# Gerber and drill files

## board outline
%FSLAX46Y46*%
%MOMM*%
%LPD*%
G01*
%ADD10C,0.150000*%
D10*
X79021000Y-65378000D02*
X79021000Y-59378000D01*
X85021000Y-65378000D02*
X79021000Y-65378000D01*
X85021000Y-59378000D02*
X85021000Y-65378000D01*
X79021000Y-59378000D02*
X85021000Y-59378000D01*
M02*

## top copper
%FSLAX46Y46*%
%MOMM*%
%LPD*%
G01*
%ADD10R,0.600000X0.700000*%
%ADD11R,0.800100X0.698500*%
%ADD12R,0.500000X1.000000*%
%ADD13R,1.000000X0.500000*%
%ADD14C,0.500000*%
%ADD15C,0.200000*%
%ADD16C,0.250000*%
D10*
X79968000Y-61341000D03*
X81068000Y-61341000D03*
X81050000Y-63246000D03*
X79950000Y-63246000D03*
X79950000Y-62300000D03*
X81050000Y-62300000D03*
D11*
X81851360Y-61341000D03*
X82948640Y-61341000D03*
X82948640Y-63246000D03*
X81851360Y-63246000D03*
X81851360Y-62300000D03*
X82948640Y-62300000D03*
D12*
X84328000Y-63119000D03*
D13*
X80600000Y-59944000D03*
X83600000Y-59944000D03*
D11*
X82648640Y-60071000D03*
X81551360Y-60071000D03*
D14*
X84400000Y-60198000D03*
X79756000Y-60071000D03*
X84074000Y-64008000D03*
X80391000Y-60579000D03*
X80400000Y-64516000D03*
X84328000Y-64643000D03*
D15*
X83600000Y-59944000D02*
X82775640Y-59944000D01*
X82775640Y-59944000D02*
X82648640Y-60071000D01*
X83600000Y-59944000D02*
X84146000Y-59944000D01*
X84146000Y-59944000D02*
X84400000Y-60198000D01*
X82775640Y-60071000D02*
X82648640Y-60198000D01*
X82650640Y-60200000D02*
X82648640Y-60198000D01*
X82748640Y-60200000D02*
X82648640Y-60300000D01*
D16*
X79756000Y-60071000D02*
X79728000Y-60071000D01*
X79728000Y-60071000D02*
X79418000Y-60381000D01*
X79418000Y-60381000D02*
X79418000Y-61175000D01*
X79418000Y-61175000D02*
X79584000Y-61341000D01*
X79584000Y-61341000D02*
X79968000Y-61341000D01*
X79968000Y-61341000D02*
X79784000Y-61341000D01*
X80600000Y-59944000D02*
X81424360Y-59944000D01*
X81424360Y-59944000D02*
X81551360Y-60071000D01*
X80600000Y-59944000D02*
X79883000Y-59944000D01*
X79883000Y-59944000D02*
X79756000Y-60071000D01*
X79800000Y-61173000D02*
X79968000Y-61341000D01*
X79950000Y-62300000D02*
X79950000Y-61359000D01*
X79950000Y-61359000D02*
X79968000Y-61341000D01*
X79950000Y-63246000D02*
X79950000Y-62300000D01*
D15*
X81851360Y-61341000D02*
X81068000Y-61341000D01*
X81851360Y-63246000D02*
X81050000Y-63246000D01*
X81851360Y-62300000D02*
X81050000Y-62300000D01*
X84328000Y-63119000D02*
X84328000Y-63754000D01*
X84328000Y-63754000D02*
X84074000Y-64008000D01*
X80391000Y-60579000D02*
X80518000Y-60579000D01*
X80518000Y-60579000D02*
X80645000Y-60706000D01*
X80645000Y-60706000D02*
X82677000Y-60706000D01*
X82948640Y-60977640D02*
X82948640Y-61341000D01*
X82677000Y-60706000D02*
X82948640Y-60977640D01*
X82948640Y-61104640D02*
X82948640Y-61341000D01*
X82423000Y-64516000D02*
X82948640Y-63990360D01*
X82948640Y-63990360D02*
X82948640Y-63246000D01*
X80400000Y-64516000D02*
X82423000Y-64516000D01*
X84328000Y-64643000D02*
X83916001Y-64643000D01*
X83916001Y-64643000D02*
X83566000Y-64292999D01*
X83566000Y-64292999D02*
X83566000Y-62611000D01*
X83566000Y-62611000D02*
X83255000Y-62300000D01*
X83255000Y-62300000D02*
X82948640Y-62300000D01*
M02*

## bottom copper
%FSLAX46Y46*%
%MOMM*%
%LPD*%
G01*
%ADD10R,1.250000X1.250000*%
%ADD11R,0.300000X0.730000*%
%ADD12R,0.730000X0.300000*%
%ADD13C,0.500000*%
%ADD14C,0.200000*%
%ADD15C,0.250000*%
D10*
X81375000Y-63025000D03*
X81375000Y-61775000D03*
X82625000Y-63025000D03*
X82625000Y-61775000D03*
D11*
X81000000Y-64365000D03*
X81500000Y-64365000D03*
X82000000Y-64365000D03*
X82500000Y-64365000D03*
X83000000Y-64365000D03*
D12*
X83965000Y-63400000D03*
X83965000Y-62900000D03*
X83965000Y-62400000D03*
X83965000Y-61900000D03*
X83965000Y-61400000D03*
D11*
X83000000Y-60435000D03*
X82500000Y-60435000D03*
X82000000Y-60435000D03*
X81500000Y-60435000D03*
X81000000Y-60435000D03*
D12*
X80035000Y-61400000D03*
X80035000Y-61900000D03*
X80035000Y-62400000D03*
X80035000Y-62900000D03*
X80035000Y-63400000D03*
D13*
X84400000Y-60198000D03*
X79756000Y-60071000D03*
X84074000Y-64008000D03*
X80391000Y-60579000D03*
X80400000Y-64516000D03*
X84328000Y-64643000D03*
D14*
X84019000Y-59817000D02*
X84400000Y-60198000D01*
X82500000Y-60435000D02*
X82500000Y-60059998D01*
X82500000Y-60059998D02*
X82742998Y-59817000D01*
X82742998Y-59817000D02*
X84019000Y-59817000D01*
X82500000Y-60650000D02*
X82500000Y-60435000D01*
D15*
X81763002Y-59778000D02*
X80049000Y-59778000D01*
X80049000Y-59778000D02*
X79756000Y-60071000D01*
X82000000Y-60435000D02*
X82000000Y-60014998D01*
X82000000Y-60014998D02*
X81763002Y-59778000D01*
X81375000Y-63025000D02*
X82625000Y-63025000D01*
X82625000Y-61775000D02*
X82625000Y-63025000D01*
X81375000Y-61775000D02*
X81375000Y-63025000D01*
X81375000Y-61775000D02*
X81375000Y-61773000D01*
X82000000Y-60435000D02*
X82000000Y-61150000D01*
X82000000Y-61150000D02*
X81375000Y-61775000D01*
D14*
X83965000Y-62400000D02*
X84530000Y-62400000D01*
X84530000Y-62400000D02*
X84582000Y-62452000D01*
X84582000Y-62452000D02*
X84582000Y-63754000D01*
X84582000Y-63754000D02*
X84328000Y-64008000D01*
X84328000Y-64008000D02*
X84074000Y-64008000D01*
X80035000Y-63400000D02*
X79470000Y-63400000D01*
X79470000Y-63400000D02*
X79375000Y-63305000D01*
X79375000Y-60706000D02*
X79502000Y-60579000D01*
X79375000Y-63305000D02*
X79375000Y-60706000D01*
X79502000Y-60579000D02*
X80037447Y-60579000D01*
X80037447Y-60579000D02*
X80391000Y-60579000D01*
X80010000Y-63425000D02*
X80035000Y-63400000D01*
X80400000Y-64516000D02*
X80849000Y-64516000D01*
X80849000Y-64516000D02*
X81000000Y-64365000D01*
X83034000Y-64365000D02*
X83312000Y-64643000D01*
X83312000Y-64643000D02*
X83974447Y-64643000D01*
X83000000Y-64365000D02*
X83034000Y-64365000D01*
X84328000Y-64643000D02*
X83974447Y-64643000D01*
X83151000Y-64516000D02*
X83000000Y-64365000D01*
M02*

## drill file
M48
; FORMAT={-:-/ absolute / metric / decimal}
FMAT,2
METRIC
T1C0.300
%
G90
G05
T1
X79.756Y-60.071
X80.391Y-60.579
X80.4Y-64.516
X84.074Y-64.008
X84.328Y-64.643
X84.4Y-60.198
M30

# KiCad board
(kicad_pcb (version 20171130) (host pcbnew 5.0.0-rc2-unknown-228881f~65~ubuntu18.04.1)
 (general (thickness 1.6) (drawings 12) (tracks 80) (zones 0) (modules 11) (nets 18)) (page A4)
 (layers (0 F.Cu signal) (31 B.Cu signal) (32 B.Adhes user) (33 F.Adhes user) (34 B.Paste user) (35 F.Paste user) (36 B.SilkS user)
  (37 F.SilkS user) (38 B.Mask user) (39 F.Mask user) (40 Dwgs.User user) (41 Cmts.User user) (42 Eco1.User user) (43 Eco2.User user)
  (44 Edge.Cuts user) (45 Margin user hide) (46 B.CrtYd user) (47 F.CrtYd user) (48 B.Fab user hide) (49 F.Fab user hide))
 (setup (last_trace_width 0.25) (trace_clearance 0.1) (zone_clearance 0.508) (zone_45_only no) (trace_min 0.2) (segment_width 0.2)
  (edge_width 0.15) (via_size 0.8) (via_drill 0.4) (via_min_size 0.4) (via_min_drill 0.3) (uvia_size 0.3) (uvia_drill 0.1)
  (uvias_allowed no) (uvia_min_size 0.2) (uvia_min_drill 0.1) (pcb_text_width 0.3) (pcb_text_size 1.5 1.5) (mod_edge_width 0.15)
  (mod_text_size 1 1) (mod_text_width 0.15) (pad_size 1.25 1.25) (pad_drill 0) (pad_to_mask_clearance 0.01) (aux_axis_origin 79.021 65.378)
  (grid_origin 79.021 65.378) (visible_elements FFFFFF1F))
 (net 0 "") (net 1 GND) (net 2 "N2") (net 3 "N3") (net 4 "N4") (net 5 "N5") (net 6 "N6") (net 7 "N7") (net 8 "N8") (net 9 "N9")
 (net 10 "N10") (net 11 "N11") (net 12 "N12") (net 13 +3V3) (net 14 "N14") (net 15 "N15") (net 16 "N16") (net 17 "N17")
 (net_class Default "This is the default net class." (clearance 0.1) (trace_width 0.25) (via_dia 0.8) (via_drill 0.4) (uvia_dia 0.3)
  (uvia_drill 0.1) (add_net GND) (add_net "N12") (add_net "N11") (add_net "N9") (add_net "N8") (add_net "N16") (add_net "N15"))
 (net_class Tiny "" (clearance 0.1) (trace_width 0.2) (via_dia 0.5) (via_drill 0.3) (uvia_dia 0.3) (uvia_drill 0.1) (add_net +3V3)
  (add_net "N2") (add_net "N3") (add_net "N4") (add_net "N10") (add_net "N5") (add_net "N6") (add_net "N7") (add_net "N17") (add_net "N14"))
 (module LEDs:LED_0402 (layer F.Cu) (at 80.518 61.341)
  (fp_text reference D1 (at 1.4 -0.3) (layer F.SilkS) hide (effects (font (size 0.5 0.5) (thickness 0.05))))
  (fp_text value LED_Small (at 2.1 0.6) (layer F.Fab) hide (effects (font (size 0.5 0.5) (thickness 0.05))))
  (pad 1 smd rect (at -0.55 0 180) (size 0.6 0.7) (layers F.Cu F.Paste F.Mask) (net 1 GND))
  (pad 2 smd rect (at 0.55 0 180) (size 0.6 0.7) (layers F.Cu F.Paste F.Mask) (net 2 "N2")))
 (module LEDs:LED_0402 (layer F.Cu) (at 80.5 63.246)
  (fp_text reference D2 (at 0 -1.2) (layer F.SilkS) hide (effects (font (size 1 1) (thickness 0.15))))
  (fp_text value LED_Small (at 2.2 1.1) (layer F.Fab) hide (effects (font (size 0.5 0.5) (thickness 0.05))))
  (pad 2 smd rect (at 0.55 0 180) (size 0.6 0.7) (layers F.Cu F.Paste F.Mask) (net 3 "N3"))
  (pad 1 smd rect (at -0.55 0 180) (size 0.6 0.7) (layers F.Cu F.Paste F.Mask) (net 1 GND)))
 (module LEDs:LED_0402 (layer F.Cu) (at 80.5 62.3)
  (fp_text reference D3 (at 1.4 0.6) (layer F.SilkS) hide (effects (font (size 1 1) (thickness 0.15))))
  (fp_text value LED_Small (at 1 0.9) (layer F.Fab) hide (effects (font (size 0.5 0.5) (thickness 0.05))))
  (pad 1 smd rect (at -0.55 0 180) (size 0.6 0.7) (layers F.Cu F.Paste F.Mask) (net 1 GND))
  (pad 2 smd rect (at 0.55 0 180) (size 0.6 0.7) (layers F.Cu F.Paste F.Mask) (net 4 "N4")))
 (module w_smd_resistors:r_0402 (layer F.Cu) (at 82.4 61.341 180)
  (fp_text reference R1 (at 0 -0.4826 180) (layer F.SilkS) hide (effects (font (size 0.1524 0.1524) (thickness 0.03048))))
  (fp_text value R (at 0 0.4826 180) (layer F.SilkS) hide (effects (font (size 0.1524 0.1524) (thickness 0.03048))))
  (pad 1 smd rect (at 0.54864 0 180) (size 0.8001 0.6985) (layers F.Cu F.Paste F.Mask) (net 2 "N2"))
  (pad 2 smd rect (at -0.54864 0 180) (size 0.8001 0.6985) (layers F.Cu F.Paste F.Mask) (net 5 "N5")))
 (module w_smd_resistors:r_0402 (layer F.Cu) (at 82.4 63.246 180)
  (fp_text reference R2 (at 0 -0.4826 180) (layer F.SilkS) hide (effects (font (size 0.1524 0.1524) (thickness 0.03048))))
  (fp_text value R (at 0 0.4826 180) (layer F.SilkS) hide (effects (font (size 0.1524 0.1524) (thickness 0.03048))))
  (pad 2 smd rect (at -0.54864 0 180) (size 0.8001 0.6985) (layers F.Cu F.Paste F.Mask) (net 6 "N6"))
  (pad 1 smd rect (at 0.54864 0 180) (size 0.8001 0.6985) (layers F.Cu F.Paste F.Mask) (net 3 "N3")))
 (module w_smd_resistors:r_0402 (layer F.Cu) (at 82.4 62.3 180)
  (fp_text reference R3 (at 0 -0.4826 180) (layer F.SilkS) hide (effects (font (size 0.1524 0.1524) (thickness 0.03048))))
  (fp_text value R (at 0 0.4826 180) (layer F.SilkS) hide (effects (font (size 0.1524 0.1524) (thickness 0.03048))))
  (pad 1 smd rect (at 0.54864 0 180) (size 0.8001 0.6985) (layers F.Cu F.Paste F.Mask) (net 4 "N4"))
  (pad 2 smd rect (at -0.54864 0 180) (size 0.8001 0.6985) (layers F.Cu F.Paste F.Mask) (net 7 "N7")))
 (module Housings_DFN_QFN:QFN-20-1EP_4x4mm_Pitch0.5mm (layer B.Cu) (at 82 62.4)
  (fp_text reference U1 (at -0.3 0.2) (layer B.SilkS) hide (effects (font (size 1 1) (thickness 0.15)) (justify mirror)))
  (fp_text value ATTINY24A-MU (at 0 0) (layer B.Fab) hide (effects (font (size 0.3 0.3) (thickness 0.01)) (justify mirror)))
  (pad 21 smd rect (at -0.625 0.625) (size 1.25 1.25) (layers B.Cu B.Paste B.Mask) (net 1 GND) (solder_paste_margin_ratio -0.2))
  (pad 21 smd rect (at -0.625 -0.625) (size 1.25 1.25) (layers B.Cu B.Paste B.Mask) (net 1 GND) (solder_paste_margin_ratio -0.2))
  (pad 21 smd rect (at 0.625 0.625) (size 1.25 1.25) (layers B.Cu B.Paste B.Mask) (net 1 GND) (solder_paste_margin_ratio -0.2))
  (pad 21 smd rect (at 0.625 -0.625) (size 1.25 1.25) (layers B.Cu B.Paste B.Mask) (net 1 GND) (solder_paste_margin_ratio -0.2))
  (pad 20 smd rect (at -1 1.965 270) (size 0.73 0.3) (layers B.Cu B.Paste B.Mask) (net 6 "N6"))
  (pad 19 smd rect (at -0.5 1.965 270) (size 0.73 0.3) (layers B.Cu B.Paste B.Mask))
  (pad 18 smd rect (at 0 1.965 270) (size 0.73 0.3) (layers B.Cu B.Paste B.Mask))
  (pad 17 smd rect (at 0.5 1.965 270) (size 0.73 0.3) (layers B.Cu B.Paste B.Mask))
  (pad 16 smd rect (at 1 1.965 270) (size 0.73 0.3) (layers B.Cu B.Paste B.Mask) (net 7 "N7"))
  (pad 15 smd rect (at 1.965 1) (size 0.73 0.3) (layers B.Cu B.Paste B.Mask) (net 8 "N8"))
  (pad 14 smd rect (at 1.965 0.5) (size 0.73 0.3) (layers B.Cu B.Paste B.Mask) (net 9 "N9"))
  (pad 13 smd rect (at 1.965 0) (size 0.73 0.3) (layers B.Cu B.Paste B.Mask) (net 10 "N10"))
  (pad 12 smd rect (at 1.965 -0.5) (size 0.73 0.3) (layers B.Cu B.Paste B.Mask) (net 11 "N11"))
  (pad 11 smd rect (at 1.965 -1) (size 0.73 0.3) (layers B.Cu B.Paste B.Mask) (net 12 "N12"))
  (pad 10 smd rect (at 1 -1.965 270) (size 0.73 0.3) (layers B.Cu B.Paste B.Mask))
  (pad 9 smd rect (at 0.5 -1.965 270) (size 0.73 0.3) (layers B.Cu B.Paste B.Mask) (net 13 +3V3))
  (pad 8 smd rect (at 0 -1.965 270) (size 0.73 0.3) (layers B.Cu B.Paste B.Mask) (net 1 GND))
  (pad 7 smd rect (at -0.5 -1.965 270) (size 0.73 0.3) (layers B.Cu B.Paste B.Mask))
  (pad 6 smd rect (at -1 -1.965 270) (size 0.73 0.3) (layers B.Cu B.Paste B.Mask))
  (pad 5 smd rect (at -1.965 -1) (size 0.73 0.3) (layers B.Cu B.Paste B.Mask) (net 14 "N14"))
  (pad 4 smd rect (at -1.965 -0.5) (size 0.73 0.3) (layers B.Cu B.Paste B.Mask) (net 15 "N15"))
  (pad 3 smd rect (at -1.965 0) (size 0.73 0.3) (layers B.Cu B.Paste B.Mask) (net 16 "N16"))
  (pad 2 smd rect (at -1.965 0.5) (size 0.73 0.3) (layers B.Cu B.Paste B.Mask) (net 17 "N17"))
  (pad 1 smd rect (at -1.965 1) (size 0.73 0.3) (layers B.Cu B.Paste B.Mask) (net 5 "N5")))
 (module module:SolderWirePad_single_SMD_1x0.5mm (layer F.Cu) (at 84.328 63.119 90)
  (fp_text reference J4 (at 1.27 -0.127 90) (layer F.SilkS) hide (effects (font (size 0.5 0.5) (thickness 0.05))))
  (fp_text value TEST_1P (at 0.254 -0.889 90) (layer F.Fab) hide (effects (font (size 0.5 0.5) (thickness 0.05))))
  (pad 1 smd rect (at 0 0 90) (size 1 0.5) (layers F.Cu F.Paste F.Mask) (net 10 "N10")))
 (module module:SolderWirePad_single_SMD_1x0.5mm (layer F.Cu) (at 80.6 59.944 180)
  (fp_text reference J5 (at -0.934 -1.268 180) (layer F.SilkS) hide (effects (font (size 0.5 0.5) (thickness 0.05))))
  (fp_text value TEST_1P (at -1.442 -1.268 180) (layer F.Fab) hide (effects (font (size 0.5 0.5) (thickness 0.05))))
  (pad 1 smd rect (at 0 0 180) (size 1 0.5) (layers F.Cu F.Paste F.Mask) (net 1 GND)))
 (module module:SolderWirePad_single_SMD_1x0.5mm (layer F.Cu) (at 83.6 59.944 180)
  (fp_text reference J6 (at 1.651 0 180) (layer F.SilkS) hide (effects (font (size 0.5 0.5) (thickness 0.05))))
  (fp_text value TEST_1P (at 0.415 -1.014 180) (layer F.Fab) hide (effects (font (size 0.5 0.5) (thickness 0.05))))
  (pad 1 smd rect (at 0 0 180) (size 1 0.5) (layers F.Cu F.Paste F.Mask) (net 13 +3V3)))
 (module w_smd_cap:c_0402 (layer F.Cu) (at 82.1 60.071)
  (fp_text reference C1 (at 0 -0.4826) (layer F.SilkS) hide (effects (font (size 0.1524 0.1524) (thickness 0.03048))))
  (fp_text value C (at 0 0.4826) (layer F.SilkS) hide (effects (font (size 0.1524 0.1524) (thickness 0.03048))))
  (pad 1 smd rect (at 0.54864 0) (size 0.8001 0.6985) (layers F.Cu F.Paste F.Mask) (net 13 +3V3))
  (pad 2 smd rect (at -0.54864 0) (size 0.8001 0.6985) (layers F.Cu F.Paste F.Mask) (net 1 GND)))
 (gr_line (start 79.021 65.378) (end 79.021 59.378) (layer Edge.Cuts) (width 0.15))
 (gr_line (start 85.021 65.378) (end 79.021 65.378) (layer Edge.Cuts) (width 0.15))
 (gr_line (start 85.021 59.378) (end 85.021 65.378) (layer Edge.Cuts) (width 0.15))
 (gr_line (start 79.021 59.378) (end 85.021 59.378) (layer Edge.Cuts) (width 0.15))
 (segment (start 83.6 59.944) (end 82.77564 59.944) (width 0.2) (layer F.Cu) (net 13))
 (segment (start 82.77564 59.944) (end 82.64864 60.071) (width 0.2) (layer F.Cu) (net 13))
 (segment (start 83.6 59.944) (end 84.146 59.944) (width 0.2) (layer F.Cu) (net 13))
 (segment (start 84.146 59.944) (end 84.4 60.198) (width 0.2) (layer F.Cu) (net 13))
 (segment (start 84.019 59.817) (end 84.4 60.198) (width 0.2) (layer B.Cu) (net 13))
 (segment (start 82.77564 60.071) (end 82.64864 60.198) (width 0.2) (layer F.Cu) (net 13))
 (segment (start 82.5 60.435) (end 82.5 60.059998) (width 0.2) (layer B.Cu) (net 13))
 (segment (start 82.5 60.059998) (end 82.742998 59.817) (width 0.2) (layer B.Cu) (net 13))
 (segment (start 82.742998 59.817) (end 84.019 59.817) (width 0.2) (layer B.Cu) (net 13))
 (segment (start 82.65064 60.2) (end 82.64864 60.198) (width 0.2) (layer F.Cu) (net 13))
 (segment (start 82.74864 60.2) (end 82.64864 60.3) (width 0.2) (layer F.Cu) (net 13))
 (segment (start 82.5 60.65) (end 82.5 60.435) (width 0.2) (layer B.Cu) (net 13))
 (via (at 84.4 60.198) (size 0.5) (drill 0.3) (layers F.Cu B.Cu) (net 13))
 (segment (start 79.756 60.071) (end 79.728 60.071) (width 0.25) (layer F.Cu) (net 1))
 (segment (start 79.728 60.071) (end 79.418 60.381) (width 0.25) (layer F.Cu) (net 1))
 (segment (start 79.418 60.381) (end 79.418 61.175) (width 0.25) (layer F.Cu) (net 1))
 (segment (start 79.418 61.175) (end 79.584 61.341) (width 0.25) (layer F.Cu) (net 1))
 (segment (start 79.584 61.341) (end 79.968 61.341) (width 0.25) (layer F.Cu) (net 1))
 (segment (start 79.968 61.341) (end 79.784 61.341) (width 0.25) (layer F.Cu) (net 1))
 (segment (start 80.6 59.944) (end 81.42436 59.944) (width 0.25) (layer F.Cu) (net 1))
 (segment (start 81.42436 59.944) (end 81.55136 60.071) (width 0.25) (layer F.Cu) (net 1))
 (segment (start 80.6 59.944) (end 79.883 59.944) (width 0.25) (layer F.Cu) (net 1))
 (segment (start 79.883 59.944) (end 79.756 60.071) (width 0.25) (layer F.Cu) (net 1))
 (segment (start 81.763002 59.778) (end 80.049 59.778) (width 0.25) (layer B.Cu) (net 1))
 (segment (start 80.049 59.778) (end 79.756 60.071) (width 0.25) (layer B.Cu) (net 1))
 (segment (start 82 60.435) (end 82 60.014998) (width 0.25) (layer B.Cu) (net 1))
 (segment (start 82 60.014998) (end 81.763002 59.778) (width 0.25) (layer B.Cu) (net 1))
 (segment (start 81.375 63.025) (end 82.625 63.025) (width 0.25) (layer B.Cu) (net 1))
 (segment (start 82.625 61.775) (end 82.625 63.025) (width 0.25) (layer B.Cu) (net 1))
 (segment (start 81.375 61.775) (end 81.375 63.025) (width 0.25) (layer B.Cu) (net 1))
 (segment (start 79.8 61.173) (end 79.968 61.341) (width 0.25) (layer F.Cu) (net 1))
 (segment (start 79.95 62.3) (end 79.95 61.359) (width 0.25) (layer F.Cu) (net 1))
 (segment (start 79.95 61.359) (end 79.968 61.341) (width 0.25) (layer F.Cu) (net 1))
 (segment (start 79.95 63.246) (end 79.95 62.3) (width 0.25) (layer F.Cu) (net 1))
 (segment (start 81.375 61.775) (end 81.375 61.773) (width 0.25) (layer B.Cu) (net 1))
 (segment (start 82 60.435) (end 82 61.15) (width 0.25) (layer B.Cu) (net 1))
 (segment (start 82 61.15) (end 81.375 61.775) (width 0.25) (layer B.Cu) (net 1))
 (via (at 79.756 60.071) (size 0.5) (drill 0.3) (layers F.Cu B.Cu) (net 1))
 (segment (start 81.85136 61.341) (end 81.068 61.341) (width 0.2) (layer F.Cu) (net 2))
 (segment (start 81.85136 63.246) (end 81.05 63.246) (width 0.2) (layer F.Cu) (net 3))
 (segment (start 81.85136 62.3) (end 81.05 62.3) (width 0.2) (layer F.Cu) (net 4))
 (segment (start 83.965 62.4) (end 84.53 62.4) (width 0.2) (layer B.Cu) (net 10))
 (segment (start 84.53 62.4) (end 84.582 62.452) (width 0.2) (layer B.Cu) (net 10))
 (segment (start 84.582 62.452) (end 84.582 63.754) (width 0.2) (layer B.Cu) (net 10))
 (segment (start 84.582 63.754) (end 84.328 64.008) (width 0.2) (layer B.Cu) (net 10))
 (segment (start 84.328 64.008) (end 84.074 64.008) (width 0.2) (layer B.Cu) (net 10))
 (segment (start 84.328 63.119) (end 84.328 63.754) (width 0.2) (layer F.Cu) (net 10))
 (segment (start 84.328 63.754) (end 84.074 64.008) (width 0.2) (layer F.Cu) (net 10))
 (via (at 84.074 64.008) (size 0.5) (drill 0.3) (layers F.Cu B.Cu) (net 10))
 (segment (start 80.035 63.4) (end 79.47 63.4) (width 0.2) (layer B.Cu) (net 5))
 (segment (start 79.47 63.4) (end 79.375 63.305) (width 0.2) (layer B.Cu) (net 5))
 (segment (start 79.375 60.706) (end 79.502 60.579) (width 0.2) (layer B.Cu) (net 5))
 (segment (start 79.375 63.305) (end 79.375 60.706) (width 0.2) (layer B.Cu) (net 5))
 (segment (start 79.502 60.579) (end 80.037447 60.579) (width 0.2) (layer B.Cu) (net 5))
 (segment (start 80.037447 60.579) (end 80.391 60.579) (width 0.2) (layer B.Cu) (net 5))
 (segment (start 80.391 60.579) (end 80.518 60.579) (width 0.2) (layer F.Cu) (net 5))
 (segment (start 80.518 60.579) (end 80.645 60.706) (width 0.2) (layer F.Cu) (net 5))
 (segment (start 80.645 60.706) (end 82.677 60.706) (width 0.2) (layer F.Cu) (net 5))
 (segment (start 82.94864 60.97764) (end 82.94864 61.341) (width 0.2) (layer F.Cu) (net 5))
 (segment (start 82.677 60.706) (end 82.94864 60.97764) (width 0.2) (layer F.Cu) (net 5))
 (segment (start 82.94864 61.10464) (end 82.94864 61.341) (width 0.2) (layer F.Cu) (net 5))
 (segment (start 80.01 63.425) (end 80.035 63.4) (width 0.2) (layer B.Cu) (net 5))
 (via (at 80.391 60.579) (size 0.5) (drill 0.3) (layers F.Cu B.Cu) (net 5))
 (segment (start 82.423 64.516) (end 82.94864 63.99036) (width 0.2) (layer F.Cu) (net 6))
 (segment (start 82.94864 63.99036) (end 82.94864 63.246) (width 0.2) (layer F.Cu) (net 6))
 (segment (start 80.4 64.516) (end 82.423 64.516) (width 0.2) (layer F.Cu) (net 6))
 (segment (start 80.4 64.516) (end 80.849 64.516) (width 0.2) (layer B.Cu) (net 6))
 (segment (start 80.849 64.516) (end 81 64.365) (width 0.2) (layer B.Cu) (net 6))
 (via (at 80.4 64.516) (size 0.5) (drill 0.3) (layers F.Cu B.Cu) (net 6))
 (segment (start 84.328 64.643) (end 83.916001 64.643) (width 0.2) (layer F.Cu) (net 7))
 (segment (start 83.916001 64.643) (end 83.566 64.292999) (width 0.2) (layer F.Cu) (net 7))
 (segment (start 83.566 64.292999) (end 83.566 62.611) (width 0.2) (layer F.Cu) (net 7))
 (segment (start 83.566 62.611) (end 83.255 62.3) (width 0.2) (layer F.Cu) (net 7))
 (segment (start 83.255 62.3) (end 82.94864 62.3) (width 0.2) (layer F.Cu) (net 7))
 (segment (start 83.034 64.365) (end 83.312 64.643) (width 0.2) (layer B.Cu) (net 7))
 (segment (start 83.312 64.643) (end 83.974447 64.643) (width 0.2) (layer B.Cu) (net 7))
 (segment (start 83 64.365) (end 83.034 64.365) (width 0.2) (layer B.Cu) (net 7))
 (segment (start 84.328 64.643) (end 83.974447 64.643) (width 0.2) (layer B.Cu) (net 7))
 (segment (start 83.151 64.516) (end 83 64.365) (width 0.2) (layer B.Cu) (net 7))
 (via (at 84.328 64.643) (size 0.5) (drill 0.3) (layers F.Cu B.Cu) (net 7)))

